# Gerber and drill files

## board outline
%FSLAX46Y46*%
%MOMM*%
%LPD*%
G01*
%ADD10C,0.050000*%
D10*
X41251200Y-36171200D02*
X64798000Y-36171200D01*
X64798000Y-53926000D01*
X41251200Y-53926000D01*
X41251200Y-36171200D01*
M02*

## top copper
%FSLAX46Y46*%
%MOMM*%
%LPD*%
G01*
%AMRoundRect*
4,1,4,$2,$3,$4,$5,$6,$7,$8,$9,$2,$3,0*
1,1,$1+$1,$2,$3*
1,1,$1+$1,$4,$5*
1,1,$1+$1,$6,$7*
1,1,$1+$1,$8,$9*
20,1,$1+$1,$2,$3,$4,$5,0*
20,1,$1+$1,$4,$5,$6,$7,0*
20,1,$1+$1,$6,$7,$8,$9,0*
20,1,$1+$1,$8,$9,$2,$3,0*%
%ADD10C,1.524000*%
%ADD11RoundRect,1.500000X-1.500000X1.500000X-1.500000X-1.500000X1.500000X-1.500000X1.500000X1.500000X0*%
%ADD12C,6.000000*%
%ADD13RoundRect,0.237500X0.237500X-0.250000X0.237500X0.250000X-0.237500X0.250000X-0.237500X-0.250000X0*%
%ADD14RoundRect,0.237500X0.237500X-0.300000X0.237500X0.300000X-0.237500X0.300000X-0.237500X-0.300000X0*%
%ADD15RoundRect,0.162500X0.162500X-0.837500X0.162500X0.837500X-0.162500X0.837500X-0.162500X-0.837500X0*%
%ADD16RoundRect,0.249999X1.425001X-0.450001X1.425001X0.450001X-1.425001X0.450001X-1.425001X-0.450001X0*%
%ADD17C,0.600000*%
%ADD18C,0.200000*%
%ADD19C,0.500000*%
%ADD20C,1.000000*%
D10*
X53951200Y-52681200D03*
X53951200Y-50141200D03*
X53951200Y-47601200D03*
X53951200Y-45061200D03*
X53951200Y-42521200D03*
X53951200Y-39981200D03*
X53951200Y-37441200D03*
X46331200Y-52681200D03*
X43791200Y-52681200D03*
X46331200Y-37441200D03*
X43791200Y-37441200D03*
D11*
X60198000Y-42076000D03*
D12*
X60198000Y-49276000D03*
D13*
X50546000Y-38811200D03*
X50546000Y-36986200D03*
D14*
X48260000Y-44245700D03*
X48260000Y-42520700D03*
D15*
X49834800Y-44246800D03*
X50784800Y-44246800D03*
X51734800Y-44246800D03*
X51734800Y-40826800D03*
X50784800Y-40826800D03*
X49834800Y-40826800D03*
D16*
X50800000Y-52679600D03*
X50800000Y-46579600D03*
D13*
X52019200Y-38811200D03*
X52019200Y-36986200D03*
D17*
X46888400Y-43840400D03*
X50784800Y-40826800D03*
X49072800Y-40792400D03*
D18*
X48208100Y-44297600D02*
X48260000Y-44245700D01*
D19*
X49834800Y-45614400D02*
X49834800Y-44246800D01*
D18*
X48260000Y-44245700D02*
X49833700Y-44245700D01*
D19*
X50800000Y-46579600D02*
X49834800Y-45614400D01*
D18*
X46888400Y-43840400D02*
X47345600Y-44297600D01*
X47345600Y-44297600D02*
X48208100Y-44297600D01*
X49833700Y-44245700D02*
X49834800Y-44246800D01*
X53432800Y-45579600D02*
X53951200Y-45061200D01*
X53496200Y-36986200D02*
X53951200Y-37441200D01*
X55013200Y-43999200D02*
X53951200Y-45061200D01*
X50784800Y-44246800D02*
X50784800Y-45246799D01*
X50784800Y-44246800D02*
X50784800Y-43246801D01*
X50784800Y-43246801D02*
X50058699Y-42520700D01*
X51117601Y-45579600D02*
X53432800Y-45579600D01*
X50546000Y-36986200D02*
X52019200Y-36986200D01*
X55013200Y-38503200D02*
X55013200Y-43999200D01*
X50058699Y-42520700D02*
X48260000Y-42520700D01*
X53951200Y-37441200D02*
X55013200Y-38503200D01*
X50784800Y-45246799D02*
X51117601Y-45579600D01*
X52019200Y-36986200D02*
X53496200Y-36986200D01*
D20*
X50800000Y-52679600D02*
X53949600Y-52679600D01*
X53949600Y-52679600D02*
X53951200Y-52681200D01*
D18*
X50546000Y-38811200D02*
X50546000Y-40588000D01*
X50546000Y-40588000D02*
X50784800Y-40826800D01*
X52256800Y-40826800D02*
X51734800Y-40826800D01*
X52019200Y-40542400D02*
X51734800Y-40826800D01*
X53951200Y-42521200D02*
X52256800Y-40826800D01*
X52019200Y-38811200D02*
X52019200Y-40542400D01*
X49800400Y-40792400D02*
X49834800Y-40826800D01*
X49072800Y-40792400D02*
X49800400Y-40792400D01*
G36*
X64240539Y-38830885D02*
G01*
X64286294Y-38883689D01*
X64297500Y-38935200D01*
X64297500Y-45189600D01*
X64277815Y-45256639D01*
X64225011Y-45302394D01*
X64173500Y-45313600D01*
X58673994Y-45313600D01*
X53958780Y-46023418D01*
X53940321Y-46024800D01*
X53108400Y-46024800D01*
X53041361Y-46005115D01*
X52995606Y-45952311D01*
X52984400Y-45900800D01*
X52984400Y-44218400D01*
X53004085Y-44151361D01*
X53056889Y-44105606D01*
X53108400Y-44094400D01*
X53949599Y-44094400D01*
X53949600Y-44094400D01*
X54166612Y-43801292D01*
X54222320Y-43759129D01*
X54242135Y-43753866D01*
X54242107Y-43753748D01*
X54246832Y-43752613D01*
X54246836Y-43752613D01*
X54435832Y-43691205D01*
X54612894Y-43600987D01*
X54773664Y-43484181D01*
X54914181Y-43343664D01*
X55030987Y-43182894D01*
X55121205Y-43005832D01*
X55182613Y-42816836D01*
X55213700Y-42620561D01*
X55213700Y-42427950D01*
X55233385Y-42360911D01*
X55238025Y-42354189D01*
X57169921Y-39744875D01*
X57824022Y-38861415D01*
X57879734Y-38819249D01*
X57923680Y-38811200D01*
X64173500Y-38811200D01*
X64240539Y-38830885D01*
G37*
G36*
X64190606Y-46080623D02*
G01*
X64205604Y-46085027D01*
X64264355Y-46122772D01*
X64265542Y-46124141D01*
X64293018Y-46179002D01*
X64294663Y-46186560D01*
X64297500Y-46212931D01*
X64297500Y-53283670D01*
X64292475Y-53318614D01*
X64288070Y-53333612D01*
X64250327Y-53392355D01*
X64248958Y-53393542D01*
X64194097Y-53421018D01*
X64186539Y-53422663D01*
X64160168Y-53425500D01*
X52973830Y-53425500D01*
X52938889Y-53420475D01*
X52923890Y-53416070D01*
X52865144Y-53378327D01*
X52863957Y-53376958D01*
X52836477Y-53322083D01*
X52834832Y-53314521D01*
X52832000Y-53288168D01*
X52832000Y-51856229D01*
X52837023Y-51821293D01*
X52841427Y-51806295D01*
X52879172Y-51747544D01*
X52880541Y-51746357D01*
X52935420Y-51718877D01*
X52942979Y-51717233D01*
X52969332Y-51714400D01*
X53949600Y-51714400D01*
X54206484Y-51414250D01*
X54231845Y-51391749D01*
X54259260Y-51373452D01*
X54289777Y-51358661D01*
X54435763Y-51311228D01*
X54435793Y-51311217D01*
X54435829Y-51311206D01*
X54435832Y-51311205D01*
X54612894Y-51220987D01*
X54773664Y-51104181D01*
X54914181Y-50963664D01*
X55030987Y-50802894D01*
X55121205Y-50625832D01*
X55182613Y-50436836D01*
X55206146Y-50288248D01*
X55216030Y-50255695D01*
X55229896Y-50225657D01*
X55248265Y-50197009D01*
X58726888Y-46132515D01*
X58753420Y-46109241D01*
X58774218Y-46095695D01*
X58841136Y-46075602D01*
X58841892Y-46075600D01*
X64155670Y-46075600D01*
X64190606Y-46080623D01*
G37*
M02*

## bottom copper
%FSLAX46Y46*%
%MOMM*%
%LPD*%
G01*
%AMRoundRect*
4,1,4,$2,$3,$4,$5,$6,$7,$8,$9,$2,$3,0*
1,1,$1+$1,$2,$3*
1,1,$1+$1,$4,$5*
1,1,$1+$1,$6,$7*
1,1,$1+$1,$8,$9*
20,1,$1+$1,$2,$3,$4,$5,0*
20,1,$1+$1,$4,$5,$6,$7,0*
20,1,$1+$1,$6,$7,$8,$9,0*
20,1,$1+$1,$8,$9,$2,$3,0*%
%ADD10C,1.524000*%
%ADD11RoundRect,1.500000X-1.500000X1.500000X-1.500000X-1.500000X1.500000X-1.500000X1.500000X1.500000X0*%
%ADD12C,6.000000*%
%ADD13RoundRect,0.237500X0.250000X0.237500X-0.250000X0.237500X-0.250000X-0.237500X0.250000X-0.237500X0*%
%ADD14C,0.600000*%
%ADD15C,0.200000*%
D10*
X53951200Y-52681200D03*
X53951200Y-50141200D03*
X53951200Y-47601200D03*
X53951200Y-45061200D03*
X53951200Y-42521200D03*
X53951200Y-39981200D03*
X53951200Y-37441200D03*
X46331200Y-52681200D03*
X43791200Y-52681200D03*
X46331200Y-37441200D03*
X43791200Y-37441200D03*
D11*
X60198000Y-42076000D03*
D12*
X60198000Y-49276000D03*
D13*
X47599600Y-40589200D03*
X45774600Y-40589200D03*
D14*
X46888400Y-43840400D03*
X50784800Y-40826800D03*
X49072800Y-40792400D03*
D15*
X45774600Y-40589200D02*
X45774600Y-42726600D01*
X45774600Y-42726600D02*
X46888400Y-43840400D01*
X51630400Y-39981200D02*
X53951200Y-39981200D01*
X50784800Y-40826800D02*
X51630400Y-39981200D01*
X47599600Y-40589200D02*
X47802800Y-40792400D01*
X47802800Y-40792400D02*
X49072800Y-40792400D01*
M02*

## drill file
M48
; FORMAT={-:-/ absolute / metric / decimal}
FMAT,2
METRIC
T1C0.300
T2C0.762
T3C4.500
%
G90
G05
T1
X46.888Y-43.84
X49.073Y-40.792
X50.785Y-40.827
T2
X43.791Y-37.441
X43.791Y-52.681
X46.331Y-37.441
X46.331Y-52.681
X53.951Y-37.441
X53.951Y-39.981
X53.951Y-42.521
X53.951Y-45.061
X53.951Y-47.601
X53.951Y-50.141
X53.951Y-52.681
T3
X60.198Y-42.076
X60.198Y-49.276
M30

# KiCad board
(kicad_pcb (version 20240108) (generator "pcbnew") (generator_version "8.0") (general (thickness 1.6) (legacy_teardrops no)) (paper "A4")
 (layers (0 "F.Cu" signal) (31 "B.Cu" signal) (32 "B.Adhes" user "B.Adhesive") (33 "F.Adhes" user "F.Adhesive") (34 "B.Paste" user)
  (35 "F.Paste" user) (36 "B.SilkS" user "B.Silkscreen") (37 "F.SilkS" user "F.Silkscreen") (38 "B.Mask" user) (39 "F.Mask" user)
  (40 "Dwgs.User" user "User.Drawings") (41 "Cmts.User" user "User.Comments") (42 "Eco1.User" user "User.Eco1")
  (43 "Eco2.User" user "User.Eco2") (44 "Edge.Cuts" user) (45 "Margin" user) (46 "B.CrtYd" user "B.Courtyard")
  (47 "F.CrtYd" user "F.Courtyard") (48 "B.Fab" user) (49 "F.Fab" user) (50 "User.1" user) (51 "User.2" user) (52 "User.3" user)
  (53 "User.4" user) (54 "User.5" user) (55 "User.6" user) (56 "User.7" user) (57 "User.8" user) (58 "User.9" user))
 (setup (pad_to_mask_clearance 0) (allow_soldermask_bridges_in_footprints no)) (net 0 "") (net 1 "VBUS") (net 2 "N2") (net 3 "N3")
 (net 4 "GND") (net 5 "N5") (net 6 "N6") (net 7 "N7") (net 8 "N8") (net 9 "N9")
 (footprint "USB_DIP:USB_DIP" (layer "F.Cu") (at 55.2212 53.9512 180)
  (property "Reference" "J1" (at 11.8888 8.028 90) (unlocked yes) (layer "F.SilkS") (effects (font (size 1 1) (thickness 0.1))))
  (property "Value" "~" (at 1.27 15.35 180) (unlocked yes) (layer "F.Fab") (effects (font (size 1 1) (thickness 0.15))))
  (pad "1" thru_hole circle (at 1.27 1.27 180) (size 1.524 1.524) (drill 0.762) (layers "*.Cu" "*.Mask") (remove_unused_layers no)
   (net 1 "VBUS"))
  (pad "2" thru_hole circle (at 1.27 3.81 180) (size 1.524 1.524) (drill 0.762) (layers "*.Cu" "*.Mask") (remove_unused_layers no)
   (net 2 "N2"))
  (pad "3" thru_hole circle (at 1.27 6.35 180) (size 1.524 1.524) (drill 0.762) (layers "*.Cu" "*.Mask") (remove_unused_layers no)
   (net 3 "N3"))
  (pad "4" thru_hole circle (at 1.27 8.89 180) (size 1.524 1.524) (drill 0.762) (layers "*.Cu" "*.Mask") (remove_unused_layers no)
   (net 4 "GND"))
  (pad "5" thru_hole circle (at 1.27 11.43 180) (size 1.524 1.524) (drill 0.762) (layers "*.Cu" "*.Mask") (remove_unused_layers no)
   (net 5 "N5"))
  (pad "6" thru_hole circle (at 1.27 13.97 180) (size 1.524 1.524) (drill 0.762) (layers "*.Cu" "*.Mask") (remove_unused_layers no)
   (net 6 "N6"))
  (pad "7" thru_hole circle (at 1.27 16.51 180) (size 1.524 1.524) (drill 0.762) (layers "*.Cu" "*.Mask") (remove_unused_layers no)
   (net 4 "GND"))
  (pad "8" thru_hole circle (at 8.89 1.27 180) (size 1.524 1.524) (drill 0.762) (layers "*.Cu" "*.Mask") (remove_unused_layers no))
  (pad "9" thru_hole circle (at 11.43 1.27 180) (size 1.524 1.524) (drill 0.762) (layers "*.Cu" "*.Mask") (remove_unused_layers no))
  (pad "10" thru_hole circle (at 8.89 16.51 180) (size 1.524 1.524) (drill 0.762) (layers "*.Cu" "*.Mask") (remove_unused_layers no))
  (pad "11" thru_hole circle (at 11.43 16.51 180) (size 1.524 1.524) (drill 0.762) (layers "*.Cu" "*.Mask") (remove_unused_layers no)))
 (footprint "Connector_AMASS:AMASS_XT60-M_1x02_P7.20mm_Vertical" (layer "F.Cu") (at 60.198 42.076 -90)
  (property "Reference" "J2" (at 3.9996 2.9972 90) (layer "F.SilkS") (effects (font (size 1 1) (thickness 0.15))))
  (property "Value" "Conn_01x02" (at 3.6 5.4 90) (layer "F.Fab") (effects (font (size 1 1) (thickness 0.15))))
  (pad "1" thru_hole roundrect (at 0 0 270) (size 6 6) (drill 4.5) (layers "*.Cu" "*.Mask") (remove_unused_layers no)
   (roundrect_rratio 0.25) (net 4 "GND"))
  (pad "2" thru_hole circle (at 7.2 0 270) (size 6 6) (drill 4.5) (layers "*.Cu" "*.Mask") (remove_unused_layers no) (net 1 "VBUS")))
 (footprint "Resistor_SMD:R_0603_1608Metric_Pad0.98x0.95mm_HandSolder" (layer "F.Cu") (at 50.546 37.8987 90)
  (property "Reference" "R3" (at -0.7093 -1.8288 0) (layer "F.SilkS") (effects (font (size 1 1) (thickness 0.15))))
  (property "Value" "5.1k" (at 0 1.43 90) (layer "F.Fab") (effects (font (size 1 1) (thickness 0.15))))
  (pad "1" smd roundrect (at -0.9125 0 90) (size 0.975 0.95) (layers "F.Cu" "F.Paste" "F.Mask") (roundrect_rratio 0.25) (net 6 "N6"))
  (pad "2" smd roundrect (at 0.9125 0 90) (size 0.975 0.95) (layers "F.Cu" "F.Paste" "F.Mask") (roundrect_rratio 0.25) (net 4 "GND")))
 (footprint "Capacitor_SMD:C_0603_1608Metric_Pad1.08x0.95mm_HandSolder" (layer "F.Cu") (at 48.26 43.3832 90)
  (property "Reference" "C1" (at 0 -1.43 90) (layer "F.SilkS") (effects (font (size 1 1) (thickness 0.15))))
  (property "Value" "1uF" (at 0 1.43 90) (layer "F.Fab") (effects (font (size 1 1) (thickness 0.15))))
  (pad "1" smd roundrect (at -0.8625 0 90) (size 1.075 0.95) (layers "F.Cu" "F.Paste" "F.Mask") (roundrect_rratio 0.25) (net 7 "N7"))
  (pad "2" smd roundrect (at 0.8625 0 90) (size 1.075 0.95) (layers "F.Cu" "F.Paste" "F.Mask") (roundrect_rratio 0.25) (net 4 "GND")))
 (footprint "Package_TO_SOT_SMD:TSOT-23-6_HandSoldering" (layer "F.Cu") (at 50.7848 42.5368 90)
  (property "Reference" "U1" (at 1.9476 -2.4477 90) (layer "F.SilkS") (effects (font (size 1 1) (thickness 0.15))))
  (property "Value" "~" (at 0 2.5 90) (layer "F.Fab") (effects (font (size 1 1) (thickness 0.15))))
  (pad "1" smd roundrect (at -1.71 -0.95 90) (size 2 0.65) (layers "F.Cu" "F.Paste" "F.Mask") (roundrect_rratio 0.25) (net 7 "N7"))
  (pad "2" smd roundrect (at -1.71 0 90) (size 2 0.65) (layers "F.Cu" "F.Paste" "F.Mask") (roundrect_rratio 0.25) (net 4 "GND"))
  (pad "3" smd roundrect (at -1.71 0.95 90) (size 2 0.65) (layers "F.Cu" "F.Paste" "F.Mask") (roundrect_rratio 0.25) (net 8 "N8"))
  (pad "4" smd roundrect (at 1.71 0.95 90) (size 2 0.65) (layers "F.Cu" "F.Paste" "F.Mask") (roundrect_rratio 0.25) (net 5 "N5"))
  (pad "5" smd roundrect (at 1.71 0 90) (size 2 0.65) (layers "F.Cu" "F.Paste" "F.Mask") (roundrect_rratio 0.25) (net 6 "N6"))
  (pad "6" smd roundrect (at 1.71 -0.95 90) (size 2 0.65) (layers "F.Cu" "F.Paste" "F.Mask") (roundrect_rratio 0.25) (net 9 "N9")))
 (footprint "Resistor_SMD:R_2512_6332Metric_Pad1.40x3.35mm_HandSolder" (layer "F.Cu") (at 50.8 49.6296 90)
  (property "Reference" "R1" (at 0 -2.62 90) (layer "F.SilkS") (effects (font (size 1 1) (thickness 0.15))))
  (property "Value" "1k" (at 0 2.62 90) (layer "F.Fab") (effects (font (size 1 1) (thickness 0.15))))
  (pad "1" smd roundrect (at -3.05 0 90) (size 1.4 3.35) (layers "F.Cu" "F.Paste" "F.Mask") (roundrect_rratio 0.178571) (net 1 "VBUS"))
  (pad "2" smd roundrect (at 3.05 0 90) (size 1.4 3.35) (layers "F.Cu" "F.Paste" "F.Mask") (roundrect_rratio 0.178571) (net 7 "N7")))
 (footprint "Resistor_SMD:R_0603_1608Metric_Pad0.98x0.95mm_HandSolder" (layer "F.Cu") (at 52.0192 37.8987 90)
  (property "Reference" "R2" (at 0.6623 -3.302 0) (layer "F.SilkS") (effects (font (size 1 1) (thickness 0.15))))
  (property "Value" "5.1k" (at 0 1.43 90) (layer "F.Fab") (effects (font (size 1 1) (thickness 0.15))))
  (pad "1" smd roundrect (at -0.9125 0 90) (size 0.975 0.95) (layers "F.Cu" "F.Paste" "F.Mask") (roundrect_rratio 0.25) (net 5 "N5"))
  (pad "2" smd roundrect (at 0.9125 0 90) (size 0.975 0.95) (layers "F.Cu" "F.Paste" "F.Mask") (roundrect_rratio 0.25) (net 4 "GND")))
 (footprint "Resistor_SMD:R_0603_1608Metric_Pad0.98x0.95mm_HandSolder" (layer "B.Cu") (at 46.6871 40.5892 180)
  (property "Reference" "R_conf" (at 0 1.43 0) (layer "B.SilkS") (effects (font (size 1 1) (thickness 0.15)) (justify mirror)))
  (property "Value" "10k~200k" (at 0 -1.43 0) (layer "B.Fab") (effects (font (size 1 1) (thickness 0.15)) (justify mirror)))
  (pad "1" smd roundrect (at -0.9125 0 180) (size 0.975 0.95) (layers "B.Cu" "B.Paste" "B.Mask") (roundrect_rratio 0.25) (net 9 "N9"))
  (pad "2" smd roundrect (at 0.9125 0 180) (size 0.975 0.95) (layers "B.Cu" "B.Paste" "B.Mask") (roundrect_rratio 0.25) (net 7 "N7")))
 (gr_rect (start 41.2512 36.1712) (end 64.798 53.926) (stroke (width 0.05) (type default)) (fill none) (layer "Edge.Cuts"))
 (segment (start 48.2081 44.2976) (end 48.26 44.2457) (width 0.2) (layer "F.Cu") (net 7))
 (segment (start 49.8348 45.6144) (end 49.8348 44.2468) (width 0.5) (layer "F.Cu") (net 7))
 (segment (start 48.26 44.2457) (end 49.8337 44.2457) (width 0.2) (layer "F.Cu") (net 7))
 (segment (start 50.8 46.5796) (end 49.8348 45.6144) (width 0.5) (layer "F.Cu") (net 7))
 (segment (start 46.8884 43.8404) (end 47.3456 44.2976) (width 0.2) (layer "F.Cu") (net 7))
 (segment (start 47.3456 44.2976) (end 48.2081 44.2976) (width 0.2) (layer "F.Cu") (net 7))
 (segment (start 49.8337 44.2457) (end 49.8348 44.2468) (width 0.2) (layer "F.Cu") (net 7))
 (via (at 46.8884 43.8404) (size 0.6) (drill 0.3) (layers "F.Cu" "B.Cu") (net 7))
 (segment (start 45.7746 40.5892) (end 45.7746 42.7266) (width 0.2) (layer "B.Cu") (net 7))
 (segment (start 45.7746 42.7266) (end 46.8884 43.8404) (width 0.2) (layer "B.Cu") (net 7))
 (segment (start 53.4328 45.5796) (end 53.9512 45.0612) (width 0.2) (layer "F.Cu") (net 4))
 (segment (start 53.4962 36.9862) (end 53.9512 37.4412) (width 0.2) (layer "F.Cu") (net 4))
 (segment (start 55.0132 43.9992) (end 53.9512 45.0612) (width 0.2) (layer "F.Cu") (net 4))
 (segment (start 50.7848 44.2468) (end 50.7848 45.246799) (width 0.2) (layer "F.Cu") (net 4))
 (segment (start 50.7848 44.2468) (end 50.7848 43.246801) (width 0.2) (layer "F.Cu") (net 4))
 (segment (start 50.7848 43.246801) (end 50.058699 42.5207) (width 0.2) (layer "F.Cu") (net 4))
 (segment (start 51.117601 45.5796) (end 53.4328 45.5796) (width 0.2) (layer "F.Cu") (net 4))
 (segment (start 50.546 36.9862) (end 52.0192 36.9862) (width 0.2) (layer "F.Cu") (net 4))
 (segment (start 55.0132 38.5032) (end 55.0132 43.9992) (width 0.2) (layer "F.Cu") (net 4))
 (segment (start 50.058699 42.5207) (end 48.26 42.5207) (width 0.2) (layer "F.Cu") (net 4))
 (segment (start 53.9512 37.4412) (end 55.0132 38.5032) (width 0.2) (layer "F.Cu") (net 4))
 (segment (start 50.7848 45.246799) (end 51.117601 45.5796) (width 0.2) (layer "F.Cu") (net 4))
 (segment (start 52.0192 36.9862) (end 53.4962 36.9862) (width 0.2) (layer "F.Cu") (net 4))
 (segment (start 50.8 52.6796) (end 53.9496 52.6796) (width 1) (layer "F.Cu") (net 1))
 (segment (start 53.9496 52.6796) (end 53.9512 52.6812) (width 1) (layer "F.Cu") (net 1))
 (segment (start 50.546 38.8112) (end 50.546 40.588) (width 0.2) (layer "F.Cu") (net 6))
 (segment (start 50.546 40.588) (end 50.7848 40.8268) (width 0.2) (layer "F.Cu") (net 6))
 (via (at 50.7848 40.8268) (size 0.6) (drill 0.3) (layers "F.Cu" "B.Cu") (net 6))
 (segment (start 51.6304 39.9812) (end 53.9512 39.9812) (width 0.2) (layer "B.Cu") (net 6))
 (segment (start 50.7848 40.8268) (end 51.6304 39.9812) (width 0.2) (layer "B.Cu") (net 6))
 (segment (start 52.2568 40.8268) (end 51.7348 40.8268) (width 0.2) (layer "F.Cu") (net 5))
 (segment (start 52.0192 40.5424) (end 51.7348 40.8268) (width 0.2) (layer "F.Cu") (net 5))
 (segment (start 53.9512 42.5212) (end 52.2568 40.8268) (width 0.2) (layer "F.Cu") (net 5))
 (segment (start 52.0192 38.8112) (end 52.0192 40.5424) (width 0.2) (layer "F.Cu") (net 5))
 (segment (start 49.8004 40.7924) (end 49.8348 40.8268) (width 0.2) (layer "F.Cu") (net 9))
 (segment (start 49.0728 40.7924) (end 49.8004 40.7924) (width 0.2) (layer "F.Cu") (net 9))
 (via (at 49.0728 40.7924) (size 0.6) (drill 0.3) (layers "F.Cu" "B.Cu") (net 9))
 (segment (start 47.5996 40.5892) (end 47.8028 40.7924) (width 0.2) (layer "B.Cu") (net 9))
 (segment (start 47.8028 40.7924) (end 49.0728 40.7924) (width 0.2) (layer "B.Cu") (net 9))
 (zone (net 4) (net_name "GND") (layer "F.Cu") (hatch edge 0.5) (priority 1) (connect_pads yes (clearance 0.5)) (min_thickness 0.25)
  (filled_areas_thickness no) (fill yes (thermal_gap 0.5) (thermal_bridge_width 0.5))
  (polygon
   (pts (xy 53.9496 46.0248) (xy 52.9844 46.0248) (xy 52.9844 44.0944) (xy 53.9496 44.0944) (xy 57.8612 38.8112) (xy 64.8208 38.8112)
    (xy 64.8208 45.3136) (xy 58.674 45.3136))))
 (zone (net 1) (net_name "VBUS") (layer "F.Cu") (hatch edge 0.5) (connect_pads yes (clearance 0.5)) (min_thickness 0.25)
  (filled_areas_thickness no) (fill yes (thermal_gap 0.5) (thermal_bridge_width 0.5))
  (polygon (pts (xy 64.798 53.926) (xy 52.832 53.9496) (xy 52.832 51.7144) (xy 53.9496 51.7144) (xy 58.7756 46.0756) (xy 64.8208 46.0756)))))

